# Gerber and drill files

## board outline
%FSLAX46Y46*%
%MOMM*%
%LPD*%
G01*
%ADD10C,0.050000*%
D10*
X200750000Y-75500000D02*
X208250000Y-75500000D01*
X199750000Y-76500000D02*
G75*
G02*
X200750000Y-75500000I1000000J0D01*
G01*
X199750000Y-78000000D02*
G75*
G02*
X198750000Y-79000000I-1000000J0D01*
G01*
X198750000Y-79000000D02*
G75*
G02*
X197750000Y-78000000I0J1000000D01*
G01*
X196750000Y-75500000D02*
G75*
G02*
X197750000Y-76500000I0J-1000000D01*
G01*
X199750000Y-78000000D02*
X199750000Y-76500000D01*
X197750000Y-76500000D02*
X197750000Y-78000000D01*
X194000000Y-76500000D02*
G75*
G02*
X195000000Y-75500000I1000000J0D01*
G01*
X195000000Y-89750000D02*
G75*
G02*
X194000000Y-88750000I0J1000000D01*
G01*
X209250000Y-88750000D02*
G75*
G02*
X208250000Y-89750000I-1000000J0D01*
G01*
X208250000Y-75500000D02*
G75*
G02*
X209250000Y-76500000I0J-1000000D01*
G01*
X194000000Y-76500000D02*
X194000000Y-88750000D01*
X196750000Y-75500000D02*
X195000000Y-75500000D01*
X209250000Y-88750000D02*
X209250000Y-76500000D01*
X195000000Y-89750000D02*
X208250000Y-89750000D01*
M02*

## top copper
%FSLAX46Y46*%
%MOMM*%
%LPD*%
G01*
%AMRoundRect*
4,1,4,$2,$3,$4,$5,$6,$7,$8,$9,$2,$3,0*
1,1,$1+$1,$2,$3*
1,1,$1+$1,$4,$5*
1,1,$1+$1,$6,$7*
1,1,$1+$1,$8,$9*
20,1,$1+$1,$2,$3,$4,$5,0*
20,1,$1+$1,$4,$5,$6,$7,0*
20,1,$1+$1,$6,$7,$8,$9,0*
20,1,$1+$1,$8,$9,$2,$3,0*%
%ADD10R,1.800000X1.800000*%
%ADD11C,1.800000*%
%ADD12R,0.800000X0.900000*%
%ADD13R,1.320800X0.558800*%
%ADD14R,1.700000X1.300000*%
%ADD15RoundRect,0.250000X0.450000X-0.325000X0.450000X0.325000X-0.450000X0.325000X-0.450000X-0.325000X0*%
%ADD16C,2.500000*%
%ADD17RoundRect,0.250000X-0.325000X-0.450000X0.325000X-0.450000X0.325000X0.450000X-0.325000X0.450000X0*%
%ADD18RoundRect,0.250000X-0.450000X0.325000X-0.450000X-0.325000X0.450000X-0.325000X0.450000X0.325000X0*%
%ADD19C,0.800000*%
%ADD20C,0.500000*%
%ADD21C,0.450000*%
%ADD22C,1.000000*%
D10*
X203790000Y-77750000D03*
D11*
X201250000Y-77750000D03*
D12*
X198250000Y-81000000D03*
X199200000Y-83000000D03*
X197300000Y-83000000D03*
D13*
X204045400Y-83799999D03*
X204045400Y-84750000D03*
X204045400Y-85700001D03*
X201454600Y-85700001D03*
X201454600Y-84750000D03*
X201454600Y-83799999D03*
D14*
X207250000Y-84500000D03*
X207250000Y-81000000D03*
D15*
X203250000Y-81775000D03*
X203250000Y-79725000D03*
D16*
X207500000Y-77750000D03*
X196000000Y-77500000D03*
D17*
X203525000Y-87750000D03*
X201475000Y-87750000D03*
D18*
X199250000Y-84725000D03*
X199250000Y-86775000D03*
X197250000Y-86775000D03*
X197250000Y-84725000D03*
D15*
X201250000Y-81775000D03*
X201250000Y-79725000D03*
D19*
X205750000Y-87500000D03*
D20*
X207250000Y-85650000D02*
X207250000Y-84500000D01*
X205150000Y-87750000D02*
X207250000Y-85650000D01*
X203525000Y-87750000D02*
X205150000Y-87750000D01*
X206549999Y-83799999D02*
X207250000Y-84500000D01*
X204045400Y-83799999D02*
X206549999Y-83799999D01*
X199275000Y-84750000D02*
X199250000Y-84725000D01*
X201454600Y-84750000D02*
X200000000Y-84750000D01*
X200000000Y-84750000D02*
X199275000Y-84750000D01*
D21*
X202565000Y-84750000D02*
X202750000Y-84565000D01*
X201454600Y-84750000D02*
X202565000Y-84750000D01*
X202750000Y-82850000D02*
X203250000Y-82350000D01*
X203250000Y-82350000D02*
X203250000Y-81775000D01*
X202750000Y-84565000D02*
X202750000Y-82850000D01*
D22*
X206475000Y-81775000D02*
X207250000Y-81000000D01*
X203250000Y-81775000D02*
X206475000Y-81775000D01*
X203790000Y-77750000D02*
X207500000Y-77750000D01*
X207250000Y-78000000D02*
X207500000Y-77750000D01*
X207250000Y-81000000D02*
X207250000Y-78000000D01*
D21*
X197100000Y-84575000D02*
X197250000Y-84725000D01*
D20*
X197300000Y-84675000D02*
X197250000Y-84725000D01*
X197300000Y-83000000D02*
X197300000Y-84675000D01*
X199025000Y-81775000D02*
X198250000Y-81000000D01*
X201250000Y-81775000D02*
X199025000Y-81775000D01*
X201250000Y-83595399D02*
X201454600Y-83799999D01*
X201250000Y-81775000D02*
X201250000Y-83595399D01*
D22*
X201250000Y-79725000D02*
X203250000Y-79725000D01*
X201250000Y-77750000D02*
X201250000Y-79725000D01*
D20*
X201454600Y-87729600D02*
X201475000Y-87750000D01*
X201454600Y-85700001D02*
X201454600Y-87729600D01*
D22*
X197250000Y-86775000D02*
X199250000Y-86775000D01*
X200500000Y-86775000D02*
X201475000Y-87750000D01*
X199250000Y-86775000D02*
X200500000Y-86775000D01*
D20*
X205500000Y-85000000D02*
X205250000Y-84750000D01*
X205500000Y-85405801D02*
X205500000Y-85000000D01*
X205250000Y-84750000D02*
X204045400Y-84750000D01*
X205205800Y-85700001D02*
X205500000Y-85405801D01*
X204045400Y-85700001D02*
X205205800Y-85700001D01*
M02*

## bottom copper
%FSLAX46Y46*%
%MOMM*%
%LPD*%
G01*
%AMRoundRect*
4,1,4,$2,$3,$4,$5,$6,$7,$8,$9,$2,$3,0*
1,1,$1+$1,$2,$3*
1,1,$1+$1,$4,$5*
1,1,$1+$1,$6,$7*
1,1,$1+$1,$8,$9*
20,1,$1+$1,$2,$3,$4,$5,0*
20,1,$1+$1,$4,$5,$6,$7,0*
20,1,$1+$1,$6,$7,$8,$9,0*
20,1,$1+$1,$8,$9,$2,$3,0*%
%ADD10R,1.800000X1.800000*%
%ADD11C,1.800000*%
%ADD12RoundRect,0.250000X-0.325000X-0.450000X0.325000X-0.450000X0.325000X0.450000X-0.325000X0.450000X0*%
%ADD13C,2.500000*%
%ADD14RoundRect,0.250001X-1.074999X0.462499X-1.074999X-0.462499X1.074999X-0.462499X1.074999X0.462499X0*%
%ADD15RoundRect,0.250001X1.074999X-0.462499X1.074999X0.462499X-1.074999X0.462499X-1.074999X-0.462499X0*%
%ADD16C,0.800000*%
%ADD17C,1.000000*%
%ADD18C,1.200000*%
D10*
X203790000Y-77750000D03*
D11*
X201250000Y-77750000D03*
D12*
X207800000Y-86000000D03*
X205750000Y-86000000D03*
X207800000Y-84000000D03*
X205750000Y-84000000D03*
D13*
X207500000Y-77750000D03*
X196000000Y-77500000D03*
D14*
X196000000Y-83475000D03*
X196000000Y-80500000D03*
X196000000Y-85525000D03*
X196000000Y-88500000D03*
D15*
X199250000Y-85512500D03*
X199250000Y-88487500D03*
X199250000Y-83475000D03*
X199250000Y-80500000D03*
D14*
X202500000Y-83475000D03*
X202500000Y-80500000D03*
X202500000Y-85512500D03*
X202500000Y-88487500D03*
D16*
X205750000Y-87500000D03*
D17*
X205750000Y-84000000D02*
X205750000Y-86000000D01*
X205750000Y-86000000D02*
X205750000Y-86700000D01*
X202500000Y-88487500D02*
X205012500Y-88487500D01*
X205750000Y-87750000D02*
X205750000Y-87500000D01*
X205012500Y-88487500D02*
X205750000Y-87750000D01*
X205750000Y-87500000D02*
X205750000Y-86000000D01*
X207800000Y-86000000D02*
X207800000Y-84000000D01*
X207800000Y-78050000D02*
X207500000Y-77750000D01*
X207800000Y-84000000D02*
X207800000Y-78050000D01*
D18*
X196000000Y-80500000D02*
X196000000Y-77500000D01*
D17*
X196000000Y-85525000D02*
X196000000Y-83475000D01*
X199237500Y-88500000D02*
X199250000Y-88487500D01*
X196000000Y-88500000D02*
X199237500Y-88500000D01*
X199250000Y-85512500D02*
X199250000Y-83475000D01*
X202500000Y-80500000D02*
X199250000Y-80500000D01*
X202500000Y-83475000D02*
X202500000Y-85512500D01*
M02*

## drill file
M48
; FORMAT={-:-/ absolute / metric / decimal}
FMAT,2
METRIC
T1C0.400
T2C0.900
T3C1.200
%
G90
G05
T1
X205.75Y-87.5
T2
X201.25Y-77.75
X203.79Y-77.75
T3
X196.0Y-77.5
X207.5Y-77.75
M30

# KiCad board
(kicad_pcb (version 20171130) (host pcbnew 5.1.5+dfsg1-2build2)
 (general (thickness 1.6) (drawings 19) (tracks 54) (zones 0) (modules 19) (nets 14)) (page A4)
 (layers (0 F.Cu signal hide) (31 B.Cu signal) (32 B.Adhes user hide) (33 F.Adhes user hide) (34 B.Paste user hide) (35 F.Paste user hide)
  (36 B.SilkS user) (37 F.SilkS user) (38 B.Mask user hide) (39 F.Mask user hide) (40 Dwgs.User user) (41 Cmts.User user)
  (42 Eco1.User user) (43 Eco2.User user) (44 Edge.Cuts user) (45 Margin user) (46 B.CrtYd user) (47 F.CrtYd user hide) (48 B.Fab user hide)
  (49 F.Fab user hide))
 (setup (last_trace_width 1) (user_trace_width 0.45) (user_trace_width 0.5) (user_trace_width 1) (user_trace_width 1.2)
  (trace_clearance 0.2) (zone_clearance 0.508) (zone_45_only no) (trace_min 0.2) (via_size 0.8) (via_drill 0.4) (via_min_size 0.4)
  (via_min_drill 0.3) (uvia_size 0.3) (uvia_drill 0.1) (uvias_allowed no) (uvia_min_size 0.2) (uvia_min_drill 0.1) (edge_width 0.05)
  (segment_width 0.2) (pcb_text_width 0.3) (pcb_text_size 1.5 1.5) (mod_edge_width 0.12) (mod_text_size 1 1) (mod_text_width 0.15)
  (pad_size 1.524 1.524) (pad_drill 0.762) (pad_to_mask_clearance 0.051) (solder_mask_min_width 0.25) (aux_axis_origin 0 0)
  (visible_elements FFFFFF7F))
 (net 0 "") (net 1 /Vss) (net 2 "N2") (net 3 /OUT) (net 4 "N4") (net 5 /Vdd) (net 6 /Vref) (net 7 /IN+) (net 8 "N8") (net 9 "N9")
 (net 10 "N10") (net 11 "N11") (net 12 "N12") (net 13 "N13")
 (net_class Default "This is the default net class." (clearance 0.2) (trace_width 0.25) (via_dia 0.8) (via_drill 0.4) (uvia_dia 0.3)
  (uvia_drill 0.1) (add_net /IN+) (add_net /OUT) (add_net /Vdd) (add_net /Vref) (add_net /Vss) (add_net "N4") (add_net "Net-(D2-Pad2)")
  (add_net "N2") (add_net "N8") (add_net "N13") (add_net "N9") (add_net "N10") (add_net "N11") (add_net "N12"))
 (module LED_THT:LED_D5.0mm (layer F.Cu) (at 203.79 77.75 180)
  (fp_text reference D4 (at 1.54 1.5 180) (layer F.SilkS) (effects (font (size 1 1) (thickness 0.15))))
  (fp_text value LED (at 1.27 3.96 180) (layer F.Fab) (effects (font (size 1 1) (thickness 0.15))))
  (pad 1 thru_hole rect (at 0 0 180) (size 1.8 1.8) (drill 0.9) (layers *.Cu *.Mask) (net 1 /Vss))
  (pad 2 thru_hole circle (at 2.54 0 180) (size 1.8 1.8) (drill 0.9) (layers *.Cu *.Mask) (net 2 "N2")))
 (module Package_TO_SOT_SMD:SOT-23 (layer F.Cu) (at 198.25 82 90)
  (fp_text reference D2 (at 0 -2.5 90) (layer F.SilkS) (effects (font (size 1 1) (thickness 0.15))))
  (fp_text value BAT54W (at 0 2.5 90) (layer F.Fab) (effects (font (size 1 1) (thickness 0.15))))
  (pad 3 smd rect (at 1 0 90) (size 0.9 0.8) (layers F.Cu F.Paste F.Mask) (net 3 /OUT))
  (pad 2 smd rect (at -1 0.95 90) (size 0.9 0.8) (layers F.Cu F.Paste F.Mask))
  (pad 1 smd rect (at -1 -0.95 90) (size 0.9 0.8) (layers F.Cu F.Paste F.Mask) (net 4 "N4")))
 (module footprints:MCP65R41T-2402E (layer F.Cu) (at 202.75 84.75)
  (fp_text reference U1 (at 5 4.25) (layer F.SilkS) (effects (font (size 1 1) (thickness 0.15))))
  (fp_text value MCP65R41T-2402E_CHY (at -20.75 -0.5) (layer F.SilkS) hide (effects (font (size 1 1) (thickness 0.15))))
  (pad 6 smd rect (at 1.2954 -0.950001) (size 1.3208 0.5588) (layers F.Cu F.Paste F.Mask) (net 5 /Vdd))
  (pad 5 smd rect (at 1.2954 0) (size 1.3208 0.5588) (layers F.Cu F.Paste F.Mask) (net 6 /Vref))
  (pad 4 smd rect (at 1.2954 0.950001) (size 1.3208 0.5588) (layers F.Cu F.Paste F.Mask) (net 6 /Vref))
  (pad 3 smd rect (at -1.2954 0.950001) (size 1.3208 0.5588) (layers F.Cu F.Paste F.Mask) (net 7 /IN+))
  (pad 2 smd rect (at -1.2954 0) (size 1.3208 0.5588) (layers F.Cu F.Paste F.Mask) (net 1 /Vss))
  (pad 1 smd rect (at -1.2954 -0.950001) (size 1.3208 0.5588) (layers F.Cu F.Paste F.Mask) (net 3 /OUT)))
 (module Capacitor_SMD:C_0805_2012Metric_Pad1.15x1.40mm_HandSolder (layer B.Cu) (at 206.775 86)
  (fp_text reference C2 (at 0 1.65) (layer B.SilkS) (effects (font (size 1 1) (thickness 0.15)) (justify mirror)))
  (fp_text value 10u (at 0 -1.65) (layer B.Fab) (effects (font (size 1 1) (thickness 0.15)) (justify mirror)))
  (pad 2 smd roundrect (at 1.025 0) (size 1.15 1.4) (layers B.Cu B.Paste B.Mask) (roundrect_rratio 0.217391) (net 1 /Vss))
  (pad 1 smd roundrect (at -1.025 0) (size 1.15 1.4) (layers B.Cu B.Paste B.Mask) (roundrect_rratio 0.217391) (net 5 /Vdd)))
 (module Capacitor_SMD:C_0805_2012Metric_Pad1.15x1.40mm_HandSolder (layer B.Cu) (at 206.775 84)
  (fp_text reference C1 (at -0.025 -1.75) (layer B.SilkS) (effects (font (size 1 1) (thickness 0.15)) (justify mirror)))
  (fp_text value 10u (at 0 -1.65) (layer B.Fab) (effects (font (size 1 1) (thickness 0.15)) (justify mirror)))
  (pad 2 smd roundrect (at 1.025 0) (size 1.15 1.4) (layers B.Cu B.Paste B.Mask) (roundrect_rratio 0.217391) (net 1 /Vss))
  (pad 1 smd roundrect (at -1.025 0) (size 1.15 1.4) (layers B.Cu B.Paste B.Mask) (roundrect_rratio 0.217391) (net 5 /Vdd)))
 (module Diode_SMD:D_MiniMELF (layer F.Cu) (at 207.25 82.75 90)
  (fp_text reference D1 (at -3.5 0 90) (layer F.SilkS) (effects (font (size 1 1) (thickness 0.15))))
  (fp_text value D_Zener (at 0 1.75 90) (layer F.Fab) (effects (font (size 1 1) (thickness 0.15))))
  (pad 1 smd rect (at -1.75 0 90) (size 1.3 1.7) (layers F.Cu F.Paste F.Mask) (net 5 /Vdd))
  (pad 2 smd rect (at 1.75 0 90) (size 1.3 1.7) (layers F.Cu F.Paste F.Mask) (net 1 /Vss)))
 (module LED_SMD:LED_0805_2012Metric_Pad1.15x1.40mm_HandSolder (layer F.Cu) (at 203.25 80.75 90)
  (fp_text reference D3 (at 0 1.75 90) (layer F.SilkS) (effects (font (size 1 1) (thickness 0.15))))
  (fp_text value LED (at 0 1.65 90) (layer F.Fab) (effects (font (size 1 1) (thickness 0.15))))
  (pad 1 smd roundrect (at -1.025 0 90) (size 1.15 1.4) (layers F.Cu F.Paste F.Mask) (roundrect_rratio 0.217391) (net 1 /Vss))
  (pad 2 smd roundrect (at 1.025 0 90) (size 1.15 1.4) (layers F.Cu F.Paste F.Mask) (roundrect_rratio 0.217391) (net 2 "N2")))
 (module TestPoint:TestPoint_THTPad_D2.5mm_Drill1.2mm (layer F.Cu) (at 207.5 77.75)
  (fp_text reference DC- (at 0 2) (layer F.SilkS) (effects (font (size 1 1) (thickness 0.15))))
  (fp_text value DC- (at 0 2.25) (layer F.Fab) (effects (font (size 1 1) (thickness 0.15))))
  (pad 1 thru_hole circle (at 0 0) (size 2.5 2.5) (drill 1.2) (layers *.Cu *.Mask) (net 1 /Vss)))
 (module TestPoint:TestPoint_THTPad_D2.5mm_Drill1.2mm (layer F.Cu) (at 196 77.5)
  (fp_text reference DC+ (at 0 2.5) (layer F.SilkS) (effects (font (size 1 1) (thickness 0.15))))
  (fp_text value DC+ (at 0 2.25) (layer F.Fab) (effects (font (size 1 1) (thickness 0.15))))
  (pad 1 thru_hole circle (at 0 0) (size 2.5 2.5) (drill 1.2) (layers *.Cu *.Mask) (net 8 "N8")))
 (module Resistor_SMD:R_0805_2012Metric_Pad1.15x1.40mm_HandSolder (layer F.Cu) (at 202.5 87.75)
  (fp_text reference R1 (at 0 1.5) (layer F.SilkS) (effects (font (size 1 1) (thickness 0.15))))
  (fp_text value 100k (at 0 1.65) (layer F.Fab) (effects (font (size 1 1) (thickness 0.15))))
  (pad 2 smd roundrect (at 1.025 0) (size 1.15 1.4) (layers F.Cu F.Paste F.Mask) (roundrect_rratio 0.217391) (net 5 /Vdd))
  (pad 1 smd roundrect (at -1.025 0) (size 1.15 1.4) (layers F.Cu F.Paste F.Mask) (roundrect_rratio 0.217391) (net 7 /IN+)))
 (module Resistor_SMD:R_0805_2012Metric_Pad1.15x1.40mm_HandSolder (layer F.Cu) (at 199.25 85.75 270)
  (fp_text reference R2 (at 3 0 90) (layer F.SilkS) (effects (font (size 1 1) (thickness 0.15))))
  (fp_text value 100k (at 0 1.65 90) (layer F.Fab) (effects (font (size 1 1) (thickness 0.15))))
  (pad 1 smd roundrect (at -1.025 0 270) (size 1.15 1.4) (layers F.Cu F.Paste F.Mask) (roundrect_rratio 0.217391) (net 1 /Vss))
  (pad 2 smd roundrect (at 1.025 0 270) (size 1.15 1.4) (layers F.Cu F.Paste F.Mask) (roundrect_rratio 0.217391) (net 7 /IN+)))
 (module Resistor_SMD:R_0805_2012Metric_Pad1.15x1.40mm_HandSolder (layer F.Cu) (at 197.25 85.75 270)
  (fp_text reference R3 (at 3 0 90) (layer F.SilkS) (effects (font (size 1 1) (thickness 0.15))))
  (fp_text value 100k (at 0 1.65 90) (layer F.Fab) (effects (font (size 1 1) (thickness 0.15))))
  (pad 2 smd roundrect (at 1.025 0 270) (size 1.15 1.4) (layers F.Cu F.Paste F.Mask) (roundrect_rratio 0.217391) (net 7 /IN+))
  (pad 1 smd roundrect (at -1.025 0 270) (size 1.15 1.4) (layers F.Cu F.Paste F.Mask) (roundrect_rratio 0.217391) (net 4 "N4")))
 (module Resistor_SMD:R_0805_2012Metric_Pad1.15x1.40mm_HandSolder (layer F.Cu) (at 201.25 80.75 90)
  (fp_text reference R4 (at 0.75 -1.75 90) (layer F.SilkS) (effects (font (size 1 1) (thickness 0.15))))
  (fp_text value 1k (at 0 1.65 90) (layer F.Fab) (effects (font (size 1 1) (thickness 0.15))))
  (pad 1 smd roundrect (at -1.025 0 90) (size 1.15 1.4) (layers F.Cu F.Paste F.Mask) (roundrect_rratio 0.217391) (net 3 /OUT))
  (pad 2 smd roundrect (at 1.025 0 90) (size 1.15 1.4) (layers F.Cu F.Paste F.Mask) (roundrect_rratio 0.217391) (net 2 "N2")))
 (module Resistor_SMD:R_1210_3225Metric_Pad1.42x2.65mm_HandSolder (layer B.Cu) (at 196 81.9875 270)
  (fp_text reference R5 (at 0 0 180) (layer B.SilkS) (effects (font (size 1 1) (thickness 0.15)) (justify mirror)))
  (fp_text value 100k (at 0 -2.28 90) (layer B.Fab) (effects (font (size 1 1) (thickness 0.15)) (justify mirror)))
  (pad 2 smd roundrect (at 1.4875 0 270) (size 1.425 2.65) (layers B.Cu B.Paste B.Mask) (roundrect_rratio 0.175439) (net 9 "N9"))
  (pad 1 smd roundrect (at -1.4875 0 270) (size 1.425 2.65) (layers B.Cu B.Paste B.Mask) (roundrect_rratio 0.175439) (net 8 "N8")))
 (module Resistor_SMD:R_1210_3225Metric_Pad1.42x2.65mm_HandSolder (layer B.Cu) (at 196 87.0125 270)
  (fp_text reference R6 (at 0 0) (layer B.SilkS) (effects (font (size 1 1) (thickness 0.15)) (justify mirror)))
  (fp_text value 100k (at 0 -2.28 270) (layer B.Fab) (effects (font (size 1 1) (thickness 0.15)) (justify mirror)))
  (pad 1 smd roundrect (at -1.4875 0 270) (size 1.425 2.65) (layers B.Cu B.Paste B.Mask) (roundrect_rratio 0.175439) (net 9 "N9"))
  (pad 2 smd roundrect (at 1.4875 0 270) (size 1.425 2.65) (layers B.Cu B.Paste B.Mask) (roundrect_rratio 0.175439) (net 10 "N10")))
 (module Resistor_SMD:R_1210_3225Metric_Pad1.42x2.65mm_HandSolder (layer B.Cu) (at 199.25 87 90)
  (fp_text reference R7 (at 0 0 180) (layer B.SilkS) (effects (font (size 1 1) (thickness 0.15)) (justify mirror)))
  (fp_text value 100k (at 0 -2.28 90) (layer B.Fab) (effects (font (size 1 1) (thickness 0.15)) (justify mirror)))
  (pad 2 smd roundrect (at 1.4875 0 90) (size 1.425 2.65) (layers B.Cu B.Paste B.Mask) (roundrect_rratio 0.175439) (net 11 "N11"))
  (pad 1 smd roundrect (at -1.4875 0 90) (size 1.425 2.65) (layers B.Cu B.Paste B.Mask) (roundrect_rratio 0.175439) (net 10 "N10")))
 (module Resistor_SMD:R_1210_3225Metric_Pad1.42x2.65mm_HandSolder (layer B.Cu) (at 199.25 81.9875 90)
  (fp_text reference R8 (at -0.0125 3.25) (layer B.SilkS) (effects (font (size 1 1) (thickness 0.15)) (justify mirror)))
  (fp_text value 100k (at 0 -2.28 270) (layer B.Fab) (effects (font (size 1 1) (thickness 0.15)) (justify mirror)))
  (pad 1 smd roundrect (at -1.4875 0 90) (size 1.425 2.65) (layers B.Cu B.Paste B.Mask) (roundrect_rratio 0.175439) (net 11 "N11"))
  (pad 2 smd roundrect (at 1.4875 0 90) (size 1.425 2.65) (layers B.Cu B.Paste B.Mask) (roundrect_rratio 0.175439) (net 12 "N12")))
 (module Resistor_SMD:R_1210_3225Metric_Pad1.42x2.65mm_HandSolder (layer B.Cu) (at 202.5 81.9875 270)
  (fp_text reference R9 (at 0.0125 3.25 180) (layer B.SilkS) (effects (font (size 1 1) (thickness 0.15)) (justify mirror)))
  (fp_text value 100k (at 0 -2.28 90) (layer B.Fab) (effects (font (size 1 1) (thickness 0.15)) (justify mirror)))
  (pad 2 smd roundrect (at 1.4875 0 270) (size 1.425 2.65) (layers B.Cu B.Paste B.Mask) (roundrect_rratio 0.175439) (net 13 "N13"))
  (pad 1 smd roundrect (at -1.4875 0 270) (size 1.425 2.65) (layers B.Cu B.Paste B.Mask) (roundrect_rratio 0.175439) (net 12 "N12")))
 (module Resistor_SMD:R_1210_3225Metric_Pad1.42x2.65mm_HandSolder (layer B.Cu) (at 202.5 87 270)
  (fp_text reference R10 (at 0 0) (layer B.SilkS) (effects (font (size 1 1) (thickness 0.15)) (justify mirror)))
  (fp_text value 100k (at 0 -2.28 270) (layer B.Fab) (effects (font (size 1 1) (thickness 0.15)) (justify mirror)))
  (pad 1 smd roundrect (at -1.4875 0 270) (size 1.425 2.65) (layers B.Cu B.Paste B.Mask) (roundrect_rratio 0.175439) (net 13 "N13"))
  (pad 2 smd roundrect (at 1.4875 0 270) (size 1.425 2.65) (layers B.Cu B.Paste B.Mask) (roundrect_rratio 0.175439) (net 5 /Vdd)))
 (gr_line (start 200.75 75.5) (end 208.25 75.5) (layer Edge.Cuts) (width 0.05))
 (gr_arc (start 200.75 76.5) (end 200.75 75.5) (angle -90) (layer Edge.Cuts) (width 0.05))
 (gr_arc (start 198.75 78) (end 198.75 79) (angle -90) (layer Edge.Cuts) (width 0.05))
 (gr_arc (start 198.75 78) (end 197.75 78) (angle -90) (layer Edge.Cuts) (width 0.05))
 (gr_arc (start 196.75 76.5) (end 197.75 76.5) (angle -90) (layer Edge.Cuts) (width 0.05))
 (gr_line (start 199.75 78) (end 199.75 76.5) (layer Edge.Cuts) (width 0.05))
 (gr_line (start 197.75 76.5) (end 197.75 78) (layer Edge.Cuts) (width 0.05))
 (gr_arc (start 195 76.5) (end 195 75.5) (angle -90) (layer Edge.Cuts) (width 0.05))
 (gr_arc (start 195 88.75) (end 194 88.75) (angle -90) (layer Edge.Cuts) (width 0.05))
 (gr_arc (start 208.25 88.75) (end 208.25 89.75) (angle -90) (layer Edge.Cuts) (width 0.05))
 (gr_arc (start 208.25 76.5) (end 209.25 76.5) (angle -90) (layer Edge.Cuts) (width 0.05))
 (gr_line (start 194 76.5) (end 194 88.75) (layer Edge.Cuts) (width 0.05))
 (gr_line (start 196.75 75.5) (end 195 75.5) (layer Edge.Cuts) (width 0.05))
 (gr_line (start 209.25 88.75) (end 209.25 76.5) (layer Edge.Cuts) (width 0.05))
 (gr_line (start 195 89.75) (end 208.25 89.75) (layer Edge.Cuts) (width 0.05))
 (segment (start 205.75 84) (end 205.75 86) (width 1) (layer B.Cu) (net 5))
 (segment (start 205.75 86) (end 205.75 86.7) (width 1) (layer B.Cu) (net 5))
 (segment (start 202.5 88.4875) (end 205.0125 88.4875) (width 1) (layer B.Cu) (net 5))
 (segment (start 205.75 87.75) (end 205.75 87.5) (width 1) (layer B.Cu) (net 5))
 (segment (start 205.0125 88.4875) (end 205.75 87.75) (width 1) (layer B.Cu) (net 5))
 (segment (start 207.25 85.65) (end 207.25 84.5) (width 0.5) (layer F.Cu) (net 5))
 (segment (start 205.15 87.75) (end 207.25 85.65) (width 0.5) (layer F.Cu) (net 5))
 (segment (start 203.525 87.75) (end 205.15 87.75) (width 0.5) (layer F.Cu) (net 5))
 (segment (start 206.549999 83.799999) (end 207.25 84.5) (width 0.5) (layer F.Cu) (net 5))
 (segment (start 204.0454 83.799999) (end 206.549999 83.799999) (width 0.5) (layer F.Cu) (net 5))
 (segment (start 205.75 87.5) (end 205.75 86) (width 1) (layer B.Cu) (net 5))
 (via (at 205.75 87.5) (size 0.8) (drill 0.4) (layers F.Cu B.Cu) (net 5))
 (segment (start 199.275 84.75) (end 199.25 84.725) (width 0.5) (layer F.Cu) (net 1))
 (segment (start 201.4546 84.75) (end 200 84.75) (width 0.5) (layer F.Cu) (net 1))
 (segment (start 200 84.75) (end 199.275 84.75) (width 0.5) (layer F.Cu) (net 1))
 (segment (start 202.565 84.75) (end 202.75 84.565) (width 0.45) (layer F.Cu) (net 1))
 (segment (start 201.4546 84.75) (end 202.565 84.75) (width 0.45) (layer F.Cu) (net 1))
 (segment (start 202.75 82.85) (end 203.25 82.35) (width 0.45) (layer F.Cu) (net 1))
 (segment (start 203.25 82.35) (end 203.25 81.775) (width 0.45) (layer F.Cu) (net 1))
 (segment (start 202.75 84.565) (end 202.75 82.85) (width 0.45) (layer F.Cu) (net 1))
 (segment (start 207.8 86) (end 207.8 84) (width 1) (layer B.Cu) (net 1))
 (segment (start 207.8 78.05) (end 207.5 77.75) (width 1) (layer B.Cu) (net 1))
 (segment (start 207.8 84) (end 207.8 78.05) (width 1) (layer B.Cu) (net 1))
 (segment (start 206.475 81.775) (end 207.25 81) (width 1) (layer F.Cu) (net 1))
 (segment (start 203.25 81.775) (end 206.475 81.775) (width 1) (layer F.Cu) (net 1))
 (segment (start 203.79 77.75) (end 207.5 77.75) (width 1) (layer F.Cu) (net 1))
 (segment (start 207.25 78) (end 207.5 77.75) (width 1) (layer F.Cu) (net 1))
 (segment (start 207.25 81) (end 207.25 78) (width 1) (layer F.Cu) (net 1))
 (segment (start 197.1 84.575) (end 197.25 84.725) (width 0.45) (layer F.Cu) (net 4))
 (segment (start 197.3 84.675) (end 197.25 84.725) (width 0.5) (layer F.Cu) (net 4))
 (segment (start 197.3 83) (end 197.3 84.675) (width 0.5) (layer F.Cu) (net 4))
 (segment (start 199.025 81.775) (end 198.25 81) (width 0.5) (layer F.Cu) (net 3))
 (segment (start 201.25 81.775) (end 199.025 81.775) (width 0.5) (layer F.Cu) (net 3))
 (segment (start 201.25 83.595399) (end 201.4546 83.799999) (width 0.5) (layer F.Cu) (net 3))
 (segment (start 201.25 81.775) (end 201.25 83.595399) (width 0.5) (layer F.Cu) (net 3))
 (segment (start 201.25 79.725) (end 203.25 79.725) (width 1) (layer F.Cu) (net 2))
 (segment (start 201.25 77.75) (end 201.25 79.725) (width 1) (layer F.Cu) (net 2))
 (segment (start 196 80.5) (end 196 77.5) (width 1.2) (layer B.Cu) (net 8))
 (segment (start 201.4546 87.7296) (end 201.475 87.75) (width 0.5) (layer F.Cu) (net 7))
 (segment (start 201.4546 85.700001) (end 201.4546 87.7296) (width 0.5) (layer F.Cu) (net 7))
 (segment (start 197.25 86.775) (end 199.25 86.775) (width 1) (layer F.Cu) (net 7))
 (segment (start 200.5 86.775) (end 201.475 87.75) (width 1) (layer F.Cu) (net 7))
 (segment (start 199.25 86.775) (end 200.5 86.775) (width 1) (layer F.Cu) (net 7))
 (segment (start 196 85.525) (end 196 83.475) (width 1) (layer B.Cu) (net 9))
 (segment (start 199.2375 88.5) (end 199.25 88.4875) (width 1) (layer B.Cu) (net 10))
 (segment (start 196 88.5) (end 199.2375 88.5) (width 1) (layer B.Cu) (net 10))
 (segment (start 199.25 85.5125) (end 199.25 83.475) (width 1) (layer B.Cu) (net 11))
 (segment (start 202.5 80.5) (end 199.25 80.5) (width 1) (layer B.Cu) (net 12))
 (segment (start 202.5 83.475) (end 202.5 85.5125) (width 1) (layer B.Cu) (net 13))
 (segment (start 205.5 85) (end 205.25 84.75) (width 0.5) (layer F.Cu) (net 6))
 (segment (start 205.5 85.405801) (end 205.5 85) (width 0.5) (layer F.Cu) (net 6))
 (segment (start 205.25 84.75) (end 204.0454 84.75) (width 0.5) (layer F.Cu) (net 6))
 (segment (start 205.2058 85.700001) (end 205.5 85.405801) (width 0.5) (layer F.Cu) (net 6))
 (segment (start 204.0454 85.700001) (end 205.2058 85.700001) (width 0.5) (layer F.Cu) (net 6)))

